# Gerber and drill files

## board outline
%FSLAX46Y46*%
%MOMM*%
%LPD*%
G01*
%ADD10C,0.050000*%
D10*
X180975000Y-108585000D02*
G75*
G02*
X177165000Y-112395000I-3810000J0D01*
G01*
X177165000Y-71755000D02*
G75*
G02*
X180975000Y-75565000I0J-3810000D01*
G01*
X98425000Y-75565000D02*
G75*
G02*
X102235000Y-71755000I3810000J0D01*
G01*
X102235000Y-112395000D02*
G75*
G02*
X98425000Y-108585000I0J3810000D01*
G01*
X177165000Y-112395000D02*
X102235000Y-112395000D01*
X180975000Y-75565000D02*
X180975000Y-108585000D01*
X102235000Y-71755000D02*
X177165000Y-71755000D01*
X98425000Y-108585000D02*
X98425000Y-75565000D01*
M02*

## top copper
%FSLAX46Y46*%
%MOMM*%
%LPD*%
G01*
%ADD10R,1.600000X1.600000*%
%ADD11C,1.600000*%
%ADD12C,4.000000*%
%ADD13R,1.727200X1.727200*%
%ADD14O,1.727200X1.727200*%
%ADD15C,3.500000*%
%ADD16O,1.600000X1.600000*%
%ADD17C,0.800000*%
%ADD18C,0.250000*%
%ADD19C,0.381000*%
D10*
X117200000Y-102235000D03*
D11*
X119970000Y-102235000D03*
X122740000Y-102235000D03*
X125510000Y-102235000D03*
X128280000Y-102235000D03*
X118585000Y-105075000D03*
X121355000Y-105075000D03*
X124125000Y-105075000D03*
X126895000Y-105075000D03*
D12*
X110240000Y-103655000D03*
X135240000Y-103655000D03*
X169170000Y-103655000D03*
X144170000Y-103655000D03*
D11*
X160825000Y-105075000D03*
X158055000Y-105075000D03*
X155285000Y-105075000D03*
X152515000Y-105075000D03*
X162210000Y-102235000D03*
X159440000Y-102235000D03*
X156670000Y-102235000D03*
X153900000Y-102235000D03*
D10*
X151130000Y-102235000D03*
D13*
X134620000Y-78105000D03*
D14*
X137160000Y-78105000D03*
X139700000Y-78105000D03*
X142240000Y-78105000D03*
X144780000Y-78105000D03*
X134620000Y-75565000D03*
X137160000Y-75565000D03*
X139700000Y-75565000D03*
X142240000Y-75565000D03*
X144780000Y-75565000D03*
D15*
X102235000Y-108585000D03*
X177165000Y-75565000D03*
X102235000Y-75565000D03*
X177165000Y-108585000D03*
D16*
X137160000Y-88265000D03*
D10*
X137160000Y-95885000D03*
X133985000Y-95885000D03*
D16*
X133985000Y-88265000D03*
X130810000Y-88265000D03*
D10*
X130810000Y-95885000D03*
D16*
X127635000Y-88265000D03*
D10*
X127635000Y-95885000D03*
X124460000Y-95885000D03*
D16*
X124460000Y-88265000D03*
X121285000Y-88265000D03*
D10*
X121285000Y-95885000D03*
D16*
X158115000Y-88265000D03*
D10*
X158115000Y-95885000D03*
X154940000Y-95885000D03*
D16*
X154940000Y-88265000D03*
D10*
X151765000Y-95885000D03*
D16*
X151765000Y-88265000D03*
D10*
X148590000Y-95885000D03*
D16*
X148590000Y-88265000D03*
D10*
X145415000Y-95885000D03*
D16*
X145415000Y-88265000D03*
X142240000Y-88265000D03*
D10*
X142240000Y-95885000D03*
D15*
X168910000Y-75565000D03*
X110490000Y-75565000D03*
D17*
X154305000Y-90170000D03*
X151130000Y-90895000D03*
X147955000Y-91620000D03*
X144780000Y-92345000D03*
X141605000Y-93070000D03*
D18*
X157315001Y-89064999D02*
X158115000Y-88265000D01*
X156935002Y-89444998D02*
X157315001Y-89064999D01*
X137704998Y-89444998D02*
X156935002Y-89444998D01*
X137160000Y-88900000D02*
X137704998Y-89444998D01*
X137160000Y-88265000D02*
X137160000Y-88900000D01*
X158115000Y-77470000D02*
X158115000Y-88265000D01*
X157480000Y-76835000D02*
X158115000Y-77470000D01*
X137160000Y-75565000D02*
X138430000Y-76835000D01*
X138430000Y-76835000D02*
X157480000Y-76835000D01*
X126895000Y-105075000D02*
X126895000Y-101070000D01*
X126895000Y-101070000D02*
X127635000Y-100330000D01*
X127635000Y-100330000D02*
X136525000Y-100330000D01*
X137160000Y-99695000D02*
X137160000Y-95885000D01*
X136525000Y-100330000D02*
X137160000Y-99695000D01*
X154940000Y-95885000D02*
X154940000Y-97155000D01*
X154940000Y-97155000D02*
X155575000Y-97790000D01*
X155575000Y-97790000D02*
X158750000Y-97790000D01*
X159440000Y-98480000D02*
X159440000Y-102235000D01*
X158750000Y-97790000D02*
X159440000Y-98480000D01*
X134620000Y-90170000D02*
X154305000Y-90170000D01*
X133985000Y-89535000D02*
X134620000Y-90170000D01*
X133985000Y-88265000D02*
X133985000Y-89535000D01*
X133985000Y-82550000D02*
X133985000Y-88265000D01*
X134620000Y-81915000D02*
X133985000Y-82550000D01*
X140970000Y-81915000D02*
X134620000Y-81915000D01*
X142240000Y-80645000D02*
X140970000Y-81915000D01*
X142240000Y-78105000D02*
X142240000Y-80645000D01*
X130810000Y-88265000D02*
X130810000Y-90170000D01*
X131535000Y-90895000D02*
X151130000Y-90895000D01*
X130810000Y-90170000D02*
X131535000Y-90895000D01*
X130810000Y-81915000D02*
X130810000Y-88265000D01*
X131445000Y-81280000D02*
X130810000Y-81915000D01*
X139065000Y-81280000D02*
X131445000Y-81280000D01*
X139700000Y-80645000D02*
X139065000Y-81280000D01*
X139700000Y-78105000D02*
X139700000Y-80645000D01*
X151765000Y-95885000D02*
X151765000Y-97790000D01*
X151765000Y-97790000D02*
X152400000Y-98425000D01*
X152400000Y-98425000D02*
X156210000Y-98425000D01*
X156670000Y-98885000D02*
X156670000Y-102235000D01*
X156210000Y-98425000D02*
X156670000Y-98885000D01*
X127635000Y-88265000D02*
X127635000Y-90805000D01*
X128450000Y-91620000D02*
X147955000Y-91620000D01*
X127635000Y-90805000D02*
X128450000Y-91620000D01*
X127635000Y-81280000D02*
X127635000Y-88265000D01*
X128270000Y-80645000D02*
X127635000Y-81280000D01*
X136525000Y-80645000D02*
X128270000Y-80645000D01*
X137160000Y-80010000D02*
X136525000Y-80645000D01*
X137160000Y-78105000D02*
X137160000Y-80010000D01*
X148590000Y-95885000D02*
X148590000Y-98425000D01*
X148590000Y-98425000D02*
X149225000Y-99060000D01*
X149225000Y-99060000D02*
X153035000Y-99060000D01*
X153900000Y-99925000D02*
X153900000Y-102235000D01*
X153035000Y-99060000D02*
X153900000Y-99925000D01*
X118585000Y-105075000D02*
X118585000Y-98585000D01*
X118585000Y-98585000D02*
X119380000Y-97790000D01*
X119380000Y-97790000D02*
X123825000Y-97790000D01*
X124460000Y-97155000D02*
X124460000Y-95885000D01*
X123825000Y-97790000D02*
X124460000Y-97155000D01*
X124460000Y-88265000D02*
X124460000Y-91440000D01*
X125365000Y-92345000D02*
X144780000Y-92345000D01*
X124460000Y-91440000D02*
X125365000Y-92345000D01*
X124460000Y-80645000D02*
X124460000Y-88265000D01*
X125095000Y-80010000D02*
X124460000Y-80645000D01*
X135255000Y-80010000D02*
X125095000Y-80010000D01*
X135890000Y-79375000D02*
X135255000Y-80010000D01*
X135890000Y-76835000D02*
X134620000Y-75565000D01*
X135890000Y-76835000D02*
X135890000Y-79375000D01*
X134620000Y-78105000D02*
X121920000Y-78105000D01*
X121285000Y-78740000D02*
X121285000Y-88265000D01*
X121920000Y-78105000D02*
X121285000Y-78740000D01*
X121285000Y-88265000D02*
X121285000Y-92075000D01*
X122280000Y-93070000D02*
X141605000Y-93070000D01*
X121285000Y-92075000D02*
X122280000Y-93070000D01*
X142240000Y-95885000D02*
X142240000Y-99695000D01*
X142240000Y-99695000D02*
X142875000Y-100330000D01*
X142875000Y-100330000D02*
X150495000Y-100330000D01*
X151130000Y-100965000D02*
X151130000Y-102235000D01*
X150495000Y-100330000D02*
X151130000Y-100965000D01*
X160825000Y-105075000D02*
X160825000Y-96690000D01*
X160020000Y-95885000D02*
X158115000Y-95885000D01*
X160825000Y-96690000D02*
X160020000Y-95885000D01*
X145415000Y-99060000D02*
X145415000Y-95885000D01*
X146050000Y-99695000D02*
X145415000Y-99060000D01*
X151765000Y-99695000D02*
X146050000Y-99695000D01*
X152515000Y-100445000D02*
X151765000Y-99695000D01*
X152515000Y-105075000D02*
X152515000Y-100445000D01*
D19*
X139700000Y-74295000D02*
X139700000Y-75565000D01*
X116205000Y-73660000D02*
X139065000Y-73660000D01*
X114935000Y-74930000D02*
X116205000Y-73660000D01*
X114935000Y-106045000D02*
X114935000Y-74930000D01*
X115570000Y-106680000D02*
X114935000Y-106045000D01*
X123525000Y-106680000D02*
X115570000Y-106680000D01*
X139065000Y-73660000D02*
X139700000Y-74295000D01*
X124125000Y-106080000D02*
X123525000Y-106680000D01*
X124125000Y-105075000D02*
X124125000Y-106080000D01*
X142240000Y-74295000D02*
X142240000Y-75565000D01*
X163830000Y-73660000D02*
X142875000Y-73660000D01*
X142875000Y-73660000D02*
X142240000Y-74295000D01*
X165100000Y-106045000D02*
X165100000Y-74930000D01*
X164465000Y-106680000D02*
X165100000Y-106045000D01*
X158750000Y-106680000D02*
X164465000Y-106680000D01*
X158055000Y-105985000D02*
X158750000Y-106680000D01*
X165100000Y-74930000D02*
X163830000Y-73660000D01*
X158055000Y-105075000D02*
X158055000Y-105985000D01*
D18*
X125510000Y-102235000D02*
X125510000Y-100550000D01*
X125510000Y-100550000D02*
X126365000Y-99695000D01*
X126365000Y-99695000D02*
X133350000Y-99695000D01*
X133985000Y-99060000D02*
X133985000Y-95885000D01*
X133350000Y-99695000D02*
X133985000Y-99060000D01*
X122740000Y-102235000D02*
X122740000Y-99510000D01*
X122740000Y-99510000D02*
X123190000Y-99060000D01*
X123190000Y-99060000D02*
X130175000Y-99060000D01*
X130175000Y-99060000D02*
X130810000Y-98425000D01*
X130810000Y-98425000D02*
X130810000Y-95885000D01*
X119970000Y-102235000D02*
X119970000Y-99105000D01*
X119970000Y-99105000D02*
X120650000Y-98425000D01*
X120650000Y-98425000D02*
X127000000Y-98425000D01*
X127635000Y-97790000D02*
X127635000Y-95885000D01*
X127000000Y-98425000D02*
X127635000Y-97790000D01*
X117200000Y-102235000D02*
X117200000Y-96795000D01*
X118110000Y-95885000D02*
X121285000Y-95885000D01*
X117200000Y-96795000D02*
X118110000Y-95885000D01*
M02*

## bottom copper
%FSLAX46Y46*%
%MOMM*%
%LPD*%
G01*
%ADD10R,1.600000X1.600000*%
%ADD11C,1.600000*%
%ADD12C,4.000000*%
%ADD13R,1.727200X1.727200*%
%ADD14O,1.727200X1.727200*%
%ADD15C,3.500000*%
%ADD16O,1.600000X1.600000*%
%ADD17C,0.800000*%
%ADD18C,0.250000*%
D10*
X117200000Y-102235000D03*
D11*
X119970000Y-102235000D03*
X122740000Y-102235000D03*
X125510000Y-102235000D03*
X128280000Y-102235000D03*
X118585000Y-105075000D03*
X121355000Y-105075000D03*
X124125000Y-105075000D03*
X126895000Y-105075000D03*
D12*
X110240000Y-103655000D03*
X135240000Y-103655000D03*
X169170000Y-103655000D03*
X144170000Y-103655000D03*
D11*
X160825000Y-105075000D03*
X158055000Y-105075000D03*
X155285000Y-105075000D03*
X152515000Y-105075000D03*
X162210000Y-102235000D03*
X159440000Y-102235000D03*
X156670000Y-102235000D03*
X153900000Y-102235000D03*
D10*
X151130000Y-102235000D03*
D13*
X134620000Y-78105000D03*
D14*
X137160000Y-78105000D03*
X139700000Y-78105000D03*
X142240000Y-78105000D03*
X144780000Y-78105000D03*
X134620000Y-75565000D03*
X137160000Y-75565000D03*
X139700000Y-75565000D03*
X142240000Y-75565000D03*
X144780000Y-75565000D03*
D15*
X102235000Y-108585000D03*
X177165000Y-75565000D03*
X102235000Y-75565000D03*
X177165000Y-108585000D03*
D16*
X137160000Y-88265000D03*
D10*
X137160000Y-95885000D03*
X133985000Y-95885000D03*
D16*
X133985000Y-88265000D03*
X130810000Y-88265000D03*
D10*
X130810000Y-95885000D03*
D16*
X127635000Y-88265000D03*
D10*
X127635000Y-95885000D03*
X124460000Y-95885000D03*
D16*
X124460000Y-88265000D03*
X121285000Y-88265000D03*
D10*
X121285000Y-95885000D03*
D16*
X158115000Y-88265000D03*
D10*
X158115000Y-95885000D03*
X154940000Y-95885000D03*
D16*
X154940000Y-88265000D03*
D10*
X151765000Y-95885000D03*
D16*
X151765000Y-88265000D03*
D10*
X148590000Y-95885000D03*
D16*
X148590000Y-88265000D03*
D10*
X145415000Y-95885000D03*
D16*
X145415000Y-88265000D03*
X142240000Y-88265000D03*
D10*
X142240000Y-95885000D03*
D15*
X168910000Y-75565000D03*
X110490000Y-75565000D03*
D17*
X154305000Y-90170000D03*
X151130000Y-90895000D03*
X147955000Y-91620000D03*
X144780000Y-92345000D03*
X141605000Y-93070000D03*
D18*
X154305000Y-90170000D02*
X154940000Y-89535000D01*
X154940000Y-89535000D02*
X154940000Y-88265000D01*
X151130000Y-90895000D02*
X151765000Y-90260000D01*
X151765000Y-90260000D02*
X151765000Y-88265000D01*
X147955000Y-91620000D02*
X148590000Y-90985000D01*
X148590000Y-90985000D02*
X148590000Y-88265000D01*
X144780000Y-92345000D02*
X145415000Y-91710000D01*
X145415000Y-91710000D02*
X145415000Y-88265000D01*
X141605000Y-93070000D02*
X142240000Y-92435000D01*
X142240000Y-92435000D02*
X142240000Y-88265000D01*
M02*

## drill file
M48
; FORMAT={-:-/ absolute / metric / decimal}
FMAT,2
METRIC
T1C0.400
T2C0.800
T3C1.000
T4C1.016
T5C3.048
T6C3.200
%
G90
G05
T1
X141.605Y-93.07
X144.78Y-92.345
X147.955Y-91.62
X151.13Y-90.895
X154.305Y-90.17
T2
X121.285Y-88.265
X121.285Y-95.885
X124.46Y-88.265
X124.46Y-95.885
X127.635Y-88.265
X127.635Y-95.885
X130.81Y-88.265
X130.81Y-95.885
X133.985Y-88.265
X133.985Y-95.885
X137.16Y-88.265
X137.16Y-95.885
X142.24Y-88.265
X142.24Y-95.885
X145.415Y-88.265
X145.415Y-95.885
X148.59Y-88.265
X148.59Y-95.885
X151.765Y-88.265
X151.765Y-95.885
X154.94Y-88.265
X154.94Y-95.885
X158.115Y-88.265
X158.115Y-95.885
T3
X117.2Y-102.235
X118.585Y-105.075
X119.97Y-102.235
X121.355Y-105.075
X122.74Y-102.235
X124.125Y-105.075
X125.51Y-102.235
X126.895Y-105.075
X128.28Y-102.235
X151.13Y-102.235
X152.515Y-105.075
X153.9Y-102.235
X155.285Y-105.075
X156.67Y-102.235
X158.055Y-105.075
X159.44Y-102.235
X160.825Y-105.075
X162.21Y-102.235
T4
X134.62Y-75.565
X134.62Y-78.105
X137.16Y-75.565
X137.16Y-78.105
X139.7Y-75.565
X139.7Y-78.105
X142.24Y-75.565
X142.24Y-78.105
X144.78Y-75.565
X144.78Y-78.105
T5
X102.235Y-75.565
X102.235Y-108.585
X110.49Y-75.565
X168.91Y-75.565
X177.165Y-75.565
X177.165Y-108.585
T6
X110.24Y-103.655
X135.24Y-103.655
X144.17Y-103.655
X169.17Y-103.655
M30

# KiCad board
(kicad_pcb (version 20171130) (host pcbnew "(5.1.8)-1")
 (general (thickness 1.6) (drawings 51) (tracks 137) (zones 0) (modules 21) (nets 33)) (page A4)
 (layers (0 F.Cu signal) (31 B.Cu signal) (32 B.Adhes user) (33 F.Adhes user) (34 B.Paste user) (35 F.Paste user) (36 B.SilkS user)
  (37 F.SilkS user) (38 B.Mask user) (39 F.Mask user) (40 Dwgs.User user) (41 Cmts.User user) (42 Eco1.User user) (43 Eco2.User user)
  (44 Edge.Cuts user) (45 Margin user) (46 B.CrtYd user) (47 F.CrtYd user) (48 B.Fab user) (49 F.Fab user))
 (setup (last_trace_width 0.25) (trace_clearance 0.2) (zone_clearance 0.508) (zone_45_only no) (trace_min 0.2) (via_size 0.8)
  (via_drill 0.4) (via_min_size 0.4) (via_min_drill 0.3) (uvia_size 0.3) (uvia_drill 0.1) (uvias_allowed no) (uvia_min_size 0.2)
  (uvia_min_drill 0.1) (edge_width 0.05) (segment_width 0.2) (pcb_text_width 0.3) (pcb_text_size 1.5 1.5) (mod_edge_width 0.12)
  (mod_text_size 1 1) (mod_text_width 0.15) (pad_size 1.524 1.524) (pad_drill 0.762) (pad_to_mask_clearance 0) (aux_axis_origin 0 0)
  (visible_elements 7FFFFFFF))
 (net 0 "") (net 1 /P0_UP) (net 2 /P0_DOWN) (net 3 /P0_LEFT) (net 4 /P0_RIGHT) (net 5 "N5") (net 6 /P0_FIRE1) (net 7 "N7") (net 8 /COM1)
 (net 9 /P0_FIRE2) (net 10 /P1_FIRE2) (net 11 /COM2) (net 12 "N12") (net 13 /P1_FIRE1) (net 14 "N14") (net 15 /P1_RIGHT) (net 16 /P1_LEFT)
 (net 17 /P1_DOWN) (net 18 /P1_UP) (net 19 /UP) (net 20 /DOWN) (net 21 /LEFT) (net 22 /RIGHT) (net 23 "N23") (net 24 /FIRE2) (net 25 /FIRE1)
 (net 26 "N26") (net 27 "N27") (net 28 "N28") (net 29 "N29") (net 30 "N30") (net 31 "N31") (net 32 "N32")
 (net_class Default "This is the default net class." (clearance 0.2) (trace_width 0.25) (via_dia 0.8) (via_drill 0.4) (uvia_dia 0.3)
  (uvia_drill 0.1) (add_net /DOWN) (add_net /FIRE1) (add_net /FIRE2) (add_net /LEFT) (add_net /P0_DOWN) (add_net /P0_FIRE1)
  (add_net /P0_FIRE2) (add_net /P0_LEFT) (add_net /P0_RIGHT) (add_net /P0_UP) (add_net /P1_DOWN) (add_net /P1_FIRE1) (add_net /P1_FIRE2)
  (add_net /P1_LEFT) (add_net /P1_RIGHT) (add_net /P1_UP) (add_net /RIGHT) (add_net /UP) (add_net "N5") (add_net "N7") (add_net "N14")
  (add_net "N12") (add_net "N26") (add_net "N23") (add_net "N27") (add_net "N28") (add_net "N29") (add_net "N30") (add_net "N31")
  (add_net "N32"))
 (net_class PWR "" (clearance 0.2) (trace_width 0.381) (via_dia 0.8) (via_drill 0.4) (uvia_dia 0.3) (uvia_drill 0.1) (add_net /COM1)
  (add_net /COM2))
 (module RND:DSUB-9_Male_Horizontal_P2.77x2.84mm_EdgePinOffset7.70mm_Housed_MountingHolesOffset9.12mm (layer F.Cu) (at 117.2 102.235)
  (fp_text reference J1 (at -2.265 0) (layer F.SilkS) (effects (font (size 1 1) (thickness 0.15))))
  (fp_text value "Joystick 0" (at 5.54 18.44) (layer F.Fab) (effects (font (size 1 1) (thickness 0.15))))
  (pad 1 thru_hole rect (at 0 0) (size 1.6 1.6) (drill 1) (layers *.Cu *.Mask) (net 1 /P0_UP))
  (pad 2 thru_hole circle (at 2.77 0) (size 1.6 1.6) (drill 1) (layers *.Cu *.Mask) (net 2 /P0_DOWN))
  (pad 3 thru_hole circle (at 5.54 0) (size 1.6 1.6) (drill 1) (layers *.Cu *.Mask) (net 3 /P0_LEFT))
  (pad 4 thru_hole circle (at 8.31 0) (size 1.6 1.6) (drill 1) (layers *.Cu *.Mask) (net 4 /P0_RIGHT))
  (pad 5 thru_hole circle (at 11.08 0) (size 1.6 1.6) (drill 1) (layers *.Cu *.Mask) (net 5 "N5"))
  (pad 6 thru_hole circle (at 1.385 2.84) (size 1.6 1.6) (drill 1) (layers *.Cu *.Mask) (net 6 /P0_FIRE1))
  (pad 7 thru_hole circle (at 4.155 2.84) (size 1.6 1.6) (drill 1) (layers *.Cu *.Mask) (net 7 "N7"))
  (pad 8 thru_hole circle (at 6.925 2.84) (size 1.6 1.6) (drill 1) (layers *.Cu *.Mask) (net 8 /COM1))
  (pad 9 thru_hole circle (at 9.695 2.84) (size 1.6 1.6) (drill 1) (layers *.Cu *.Mask) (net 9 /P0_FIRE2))
  (pad 0 thru_hole circle (at -6.96 1.42) (size 4 4) (drill 3.2) (layers *.Cu *.Mask))
  (pad 0 thru_hole circle (at 18.04 1.42) (size 4 4) (drill 3.2) (layers *.Cu *.Mask)))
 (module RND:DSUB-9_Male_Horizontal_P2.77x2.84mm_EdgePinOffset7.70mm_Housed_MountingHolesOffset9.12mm (layer F.Cu) (at 151.13 102.235)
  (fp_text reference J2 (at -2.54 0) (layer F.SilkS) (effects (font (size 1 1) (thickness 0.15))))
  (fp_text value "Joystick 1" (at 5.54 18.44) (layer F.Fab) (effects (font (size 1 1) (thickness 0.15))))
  (pad 0 thru_hole circle (at 18.04 1.42) (size 4 4) (drill 3.2) (layers *.Cu *.Mask))
  (pad 0 thru_hole circle (at -6.96 1.42) (size 4 4) (drill 3.2) (layers *.Cu *.Mask))
  (pad 9 thru_hole circle (at 9.695 2.84) (size 1.6 1.6) (drill 1) (layers *.Cu *.Mask) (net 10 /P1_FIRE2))
  (pad 8 thru_hole circle (at 6.925 2.84) (size 1.6 1.6) (drill 1) (layers *.Cu *.Mask) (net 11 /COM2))
  (pad 7 thru_hole circle (at 4.155 2.84) (size 1.6 1.6) (drill 1) (layers *.Cu *.Mask) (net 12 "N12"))
  (pad 6 thru_hole circle (at 1.385 2.84) (size 1.6 1.6) (drill 1) (layers *.Cu *.Mask) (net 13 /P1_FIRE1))
  (pad 5 thru_hole circle (at 11.08 0) (size 1.6 1.6) (drill 1) (layers *.Cu *.Mask) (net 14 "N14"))
  (pad 4 thru_hole circle (at 8.31 0) (size 1.6 1.6) (drill 1) (layers *.Cu *.Mask) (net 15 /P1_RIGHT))
  (pad 3 thru_hole circle (at 5.54 0) (size 1.6 1.6) (drill 1) (layers *.Cu *.Mask) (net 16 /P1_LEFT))
  (pad 2 thru_hole circle (at 2.77 0) (size 1.6 1.6) (drill 1) (layers *.Cu *.Mask) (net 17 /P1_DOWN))
  (pad 1 thru_hole rect (at 0 0) (size 1.6 1.6) (drill 1) (layers *.Cu *.Mask) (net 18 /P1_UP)))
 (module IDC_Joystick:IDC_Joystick (layer F.Cu) (at 134.62 78.105 90)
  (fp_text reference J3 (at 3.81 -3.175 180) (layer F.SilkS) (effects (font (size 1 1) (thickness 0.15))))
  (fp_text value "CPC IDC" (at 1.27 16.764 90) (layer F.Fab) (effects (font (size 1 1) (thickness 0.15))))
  (pad 1 thru_hole rect (at 0 0 90) (size 1.7272 1.7272) (drill 1.016) (layers *.Cu *.Mask) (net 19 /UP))
  (pad 2 thru_hole oval (at 0 2.54 90) (size 1.7272 1.7272) (drill 1.016) (layers *.Cu *.Mask) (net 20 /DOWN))
  (pad 3 thru_hole oval (at 0 5.08 90) (size 1.7272 1.7272) (drill 1.016) (layers *.Cu *.Mask) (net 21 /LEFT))
  (pad 4 thru_hole oval (at 0 7.62 90) (size 1.7272 1.7272) (drill 1.016) (layers *.Cu *.Mask) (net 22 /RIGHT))
  (pad 5 thru_hole oval (at 0 10.16 90) (size 1.7272 1.7272) (drill 1.016) (layers *.Cu *.Mask) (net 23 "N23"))
  (pad 6 thru_hole oval (at 2.54 0 90) (size 1.7272 1.7272) (drill 1.016) (layers *.Cu *.Mask) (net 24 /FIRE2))
  (pad 7 thru_hole oval (at 2.54 2.54 90) (size 1.7272 1.7272) (drill 1.016) (layers *.Cu *.Mask) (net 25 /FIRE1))
  (pad 8 thru_hole oval (at 2.54 5.08 90) (size 1.7272 1.7272) (drill 1.016) (layers *.Cu *.Mask) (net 8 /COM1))
  (pad 9 thru_hole oval (at 2.54 7.62 90) (size 1.7272 1.7272) (drill 1.016) (layers *.Cu *.Mask) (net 11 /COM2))
  (pad 10 thru_hole oval (at 2.54 10.16 90) (size 1.7272 1.7272) (drill 1.016) (layers *.Cu *.Mask) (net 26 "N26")))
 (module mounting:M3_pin (layer F.Cu) (at 102.235 108.585)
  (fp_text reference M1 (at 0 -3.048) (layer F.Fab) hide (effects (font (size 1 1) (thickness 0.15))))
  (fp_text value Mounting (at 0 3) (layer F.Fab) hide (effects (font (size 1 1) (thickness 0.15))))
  (pad 1 thru_hole circle (at 0 0) (size 3.5 3.5) (drill 3.048) (layers *.Cu *.Mask) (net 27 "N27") (solder_mask_margin 0.8)))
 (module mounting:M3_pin (layer F.Cu) (at 177.165 75.565)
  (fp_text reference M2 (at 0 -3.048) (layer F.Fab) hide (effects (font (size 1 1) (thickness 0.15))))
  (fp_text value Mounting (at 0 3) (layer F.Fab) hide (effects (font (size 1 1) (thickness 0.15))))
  (pad 1 thru_hole circle (at 0 0) (size 3.5 3.5) (drill 3.048) (layers *.Cu *.Mask) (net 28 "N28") (solder_mask_margin 0.8)))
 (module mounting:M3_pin (layer F.Cu) (at 102.235 75.565)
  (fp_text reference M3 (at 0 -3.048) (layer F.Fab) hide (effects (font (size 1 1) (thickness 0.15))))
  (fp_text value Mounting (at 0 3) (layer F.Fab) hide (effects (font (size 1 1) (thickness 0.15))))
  (pad 1 thru_hole circle (at 0 0) (size 3.5 3.5) (drill 3.048) (layers *.Cu *.Mask) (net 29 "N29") (solder_mask_margin 0.8)))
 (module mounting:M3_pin (layer F.Cu) (at 177.165 108.585)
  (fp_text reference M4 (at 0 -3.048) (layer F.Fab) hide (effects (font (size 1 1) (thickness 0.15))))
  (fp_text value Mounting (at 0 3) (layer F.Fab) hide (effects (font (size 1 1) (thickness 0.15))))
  (pad 1 thru_hole circle (at 0 0) (size 3.5 3.5) (drill 3.048) (layers *.Cu *.Mask) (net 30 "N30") (solder_mask_margin 0.8)))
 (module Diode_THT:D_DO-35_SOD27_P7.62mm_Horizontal (layer F.Cu) (at 137.16 95.885 90)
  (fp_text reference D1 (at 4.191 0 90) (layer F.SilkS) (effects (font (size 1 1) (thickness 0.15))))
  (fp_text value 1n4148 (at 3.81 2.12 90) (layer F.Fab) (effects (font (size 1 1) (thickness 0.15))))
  (pad 2 thru_hole oval (at 7.62 0 90) (size 1.6 1.6) (drill 0.8) (layers *.Cu *.Mask) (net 25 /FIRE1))
  (pad 1 thru_hole rect (at 0 0 90) (size 1.6 1.6) (drill 0.8) (layers *.Cu *.Mask) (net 9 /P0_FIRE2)))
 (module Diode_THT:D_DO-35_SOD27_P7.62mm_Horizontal (layer F.Cu) (at 133.985 95.885 90)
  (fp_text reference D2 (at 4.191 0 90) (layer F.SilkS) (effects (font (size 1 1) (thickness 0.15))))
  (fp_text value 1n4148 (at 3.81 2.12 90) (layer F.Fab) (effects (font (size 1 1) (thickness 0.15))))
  (pad 1 thru_hole rect (at 0 0 90) (size 1.6 1.6) (drill 0.8) (layers *.Cu *.Mask) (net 4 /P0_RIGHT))
  (pad 2 thru_hole oval (at 7.62 0 90) (size 1.6 1.6) (drill 0.8) (layers *.Cu *.Mask) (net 22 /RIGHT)))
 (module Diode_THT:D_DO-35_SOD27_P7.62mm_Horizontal (layer F.Cu) (at 130.81 95.885 90)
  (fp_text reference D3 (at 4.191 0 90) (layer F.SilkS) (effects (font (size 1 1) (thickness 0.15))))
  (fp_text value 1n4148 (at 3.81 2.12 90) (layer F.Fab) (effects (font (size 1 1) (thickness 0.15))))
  (pad 2 thru_hole oval (at 7.62 0 90) (size 1.6 1.6) (drill 0.8) (layers *.Cu *.Mask) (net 21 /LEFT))
  (pad 1 thru_hole rect (at 0 0 90) (size 1.6 1.6) (drill 0.8) (layers *.Cu *.Mask) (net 3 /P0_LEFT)))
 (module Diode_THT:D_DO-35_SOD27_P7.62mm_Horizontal (layer F.Cu) (at 127.635 95.885 90)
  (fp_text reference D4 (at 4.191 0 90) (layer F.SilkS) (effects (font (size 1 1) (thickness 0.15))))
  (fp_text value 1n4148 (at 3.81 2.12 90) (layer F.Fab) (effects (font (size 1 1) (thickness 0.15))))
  (pad 2 thru_hole oval (at 7.62 0 90) (size 1.6 1.6) (drill 0.8) (layers *.Cu *.Mask) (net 20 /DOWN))
  (pad 1 thru_hole rect (at 0 0 90) (size 1.6 1.6) (drill 0.8) (layers *.Cu *.Mask) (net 2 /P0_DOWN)))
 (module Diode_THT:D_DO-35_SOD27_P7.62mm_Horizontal (layer F.Cu) (at 124.46 95.885 90)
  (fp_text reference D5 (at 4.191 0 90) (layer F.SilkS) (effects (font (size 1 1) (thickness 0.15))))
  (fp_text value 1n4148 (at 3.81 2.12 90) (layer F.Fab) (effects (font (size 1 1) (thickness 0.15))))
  (pad 1 thru_hole rect (at 0 0 90) (size 1.6 1.6) (drill 0.8) (layers *.Cu *.Mask) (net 6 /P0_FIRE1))
  (pad 2 thru_hole oval (at 7.62 0 90) (size 1.6 1.6) (drill 0.8) (layers *.Cu *.Mask) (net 24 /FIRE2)))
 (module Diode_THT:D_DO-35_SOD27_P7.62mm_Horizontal (layer F.Cu) (at 121.285 95.885 90)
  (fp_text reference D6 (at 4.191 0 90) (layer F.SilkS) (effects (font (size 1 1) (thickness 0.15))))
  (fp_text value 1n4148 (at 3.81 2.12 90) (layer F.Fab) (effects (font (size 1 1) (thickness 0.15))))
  (pad 2 thru_hole oval (at 7.62 0 90) (size 1.6 1.6) (drill 0.8) (layers *.Cu *.Mask) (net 19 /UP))
  (pad 1 thru_hole rect (at 0 0 90) (size 1.6 1.6) (drill 0.8) (layers *.Cu *.Mask) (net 1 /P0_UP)))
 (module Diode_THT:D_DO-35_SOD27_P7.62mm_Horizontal (layer F.Cu) (at 158.115 95.885 90)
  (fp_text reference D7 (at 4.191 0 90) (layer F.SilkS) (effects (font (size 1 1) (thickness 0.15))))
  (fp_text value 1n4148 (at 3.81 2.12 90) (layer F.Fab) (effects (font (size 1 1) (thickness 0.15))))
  (pad 2 thru_hole oval (at 7.62 0 90) (size 1.6 1.6) (drill 0.8) (layers *.Cu *.Mask) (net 25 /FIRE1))
  (pad 1 thru_hole rect (at 0 0 90) (size 1.6 1.6) (drill 0.8) (layers *.Cu *.Mask) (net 10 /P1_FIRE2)))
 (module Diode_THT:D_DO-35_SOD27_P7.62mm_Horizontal (layer F.Cu) (at 154.94 95.885 90)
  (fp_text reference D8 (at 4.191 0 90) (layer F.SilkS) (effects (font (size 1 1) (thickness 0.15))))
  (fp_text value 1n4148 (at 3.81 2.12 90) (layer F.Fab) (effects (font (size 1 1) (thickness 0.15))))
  (pad 1 thru_hole rect (at 0 0 90) (size 1.6 1.6) (drill 0.8) (layers *.Cu *.Mask) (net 15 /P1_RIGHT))
  (pad 2 thru_hole oval (at 7.62 0 90) (size 1.6 1.6) (drill 0.8) (layers *.Cu *.Mask) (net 22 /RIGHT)))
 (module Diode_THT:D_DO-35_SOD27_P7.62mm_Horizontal (layer F.Cu) (at 151.765 95.885 90)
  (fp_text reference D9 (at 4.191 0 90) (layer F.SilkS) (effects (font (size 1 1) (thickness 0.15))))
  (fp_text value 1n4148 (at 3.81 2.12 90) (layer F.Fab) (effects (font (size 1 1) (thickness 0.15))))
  (pad 1 thru_hole rect (at 0 0 90) (size 1.6 1.6) (drill 0.8) (layers *.Cu *.Mask) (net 16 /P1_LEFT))
  (pad 2 thru_hole oval (at 7.62 0 90) (size 1.6 1.6) (drill 0.8) (layers *.Cu *.Mask) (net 21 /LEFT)))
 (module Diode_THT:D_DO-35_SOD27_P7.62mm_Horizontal (layer F.Cu) (at 148.59 95.885 90)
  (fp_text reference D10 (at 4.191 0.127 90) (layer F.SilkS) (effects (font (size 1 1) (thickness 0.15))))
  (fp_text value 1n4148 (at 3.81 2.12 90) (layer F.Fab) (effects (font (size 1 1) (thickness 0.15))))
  (pad 1 thru_hole rect (at 0 0 90) (size 1.6 1.6) (drill 0.8) (layers *.Cu *.Mask) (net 17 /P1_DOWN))
  (pad 2 thru_hole oval (at 7.62 0 90) (size 1.6 1.6) (drill 0.8) (layers *.Cu *.Mask) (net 20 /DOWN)))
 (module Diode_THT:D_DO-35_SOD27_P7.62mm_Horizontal (layer F.Cu) (at 145.415 95.885 90)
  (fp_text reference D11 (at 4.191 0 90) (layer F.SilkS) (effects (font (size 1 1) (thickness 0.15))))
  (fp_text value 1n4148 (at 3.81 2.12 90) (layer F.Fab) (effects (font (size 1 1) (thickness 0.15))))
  (pad 1 thru_hole rect (at 0 0 90) (size 1.6 1.6) (drill 0.8) (layers *.Cu *.Mask) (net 13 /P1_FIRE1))
  (pad 2 thru_hole oval (at 7.62 0 90) (size 1.6 1.6) (drill 0.8) (layers *.Cu *.Mask) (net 24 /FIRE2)))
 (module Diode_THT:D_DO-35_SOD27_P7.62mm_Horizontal (layer F.Cu) (at 142.24 95.885 90)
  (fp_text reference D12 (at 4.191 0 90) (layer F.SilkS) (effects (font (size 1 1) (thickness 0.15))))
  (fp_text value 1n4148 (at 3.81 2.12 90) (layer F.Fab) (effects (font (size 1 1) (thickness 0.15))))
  (pad 2 thru_hole oval (at 7.62 0 90) (size 1.6 1.6) (drill 0.8) (layers *.Cu *.Mask) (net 19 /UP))
  (pad 1 thru_hole rect (at 0 0 90) (size 1.6 1.6) (drill 0.8) (layers *.Cu *.Mask) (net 18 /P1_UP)))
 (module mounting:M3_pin (layer F.Cu) (at 168.91 75.565)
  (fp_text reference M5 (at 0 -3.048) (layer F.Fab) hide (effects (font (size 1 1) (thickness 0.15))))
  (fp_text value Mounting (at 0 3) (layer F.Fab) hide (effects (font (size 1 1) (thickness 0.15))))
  (pad 1 thru_hole circle (at 0 0) (size 3.5 3.5) (drill 3.048) (layers *.Cu *.Mask) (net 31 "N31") (solder_mask_margin 0.8)))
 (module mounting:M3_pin (layer F.Cu) (at 110.49 75.565)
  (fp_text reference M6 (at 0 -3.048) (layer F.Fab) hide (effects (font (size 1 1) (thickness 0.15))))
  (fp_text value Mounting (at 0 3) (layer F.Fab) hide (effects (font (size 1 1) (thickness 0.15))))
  (pad 1 thru_hole circle (at 0 0) (size 3.5 3.5) (drill 3.048) (layers *.Cu *.Mask) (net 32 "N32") (solder_mask_margin 0.8)))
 (gr_arc (start 177.165 108.585) (end 177.165 112.395) (angle -90) (layer Edge.Cuts) (width 0.05))
 (gr_arc (start 177.165 75.565) (end 180.975 75.565) (angle -90) (layer Edge.Cuts) (width 0.05))
 (gr_arc (start 102.235 75.565) (end 102.235 71.755) (angle -90) (layer Edge.Cuts) (width 0.05))
 (gr_arc (start 102.235 108.585) (end 98.425 108.585) (angle -90) (layer Edge.Cuts) (width 0.05))
 (gr_line (start 177.165 112.395) (end 102.235 112.395) (layer Edge.Cuts) (width 0.05))
 (gr_line (start 180.975 75.565) (end 180.975 108.585) (layer Edge.Cuts) (width 0.05))
 (gr_line (start 102.235 71.755) (end 177.165 71.755) (layer Edge.Cuts) (width 0.05))
 (gr_line (start 98.425 108.585) (end 98.425 75.565) (layer Edge.Cuts) (width 0.05))
 (segment (start 157.315001 89.064999) (end 158.115 88.265) (width 0.25) (layer F.Cu) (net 25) (status 20))
 (segment (start 156.935002 89.444998) (end 157.315001 89.064999) (width 0.25) (layer F.Cu) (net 25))
 (segment (start 137.704998 89.444998) (end 156.935002 89.444998) (width 0.25) (layer F.Cu) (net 25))
 (segment (start 137.16 88.9) (end 137.704998 89.444998) (width 0.25) (layer F.Cu) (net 25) (status 10))
 (segment (start 137.16 88.265) (end 137.16 88.9) (width 0.25) (layer F.Cu) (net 25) (status 30))
 (segment (start 158.115 77.47) (end 158.115 88.265) (width 0.25) (layer F.Cu) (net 25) (status 20))
 (segment (start 157.48 76.835) (end 158.115 77.47) (width 0.25) (layer F.Cu) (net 25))
 (segment (start 137.16 75.565) (end 138.43 76.835) (width 0.25) (layer F.Cu) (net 25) (status 10))
 (segment (start 138.43 76.835) (end 157.48 76.835) (width 0.25) (layer F.Cu) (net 25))
 (segment (start 126.895 105.075) (end 126.895 101.07) (width 0.25) (layer F.Cu) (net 9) (status 10))
 (segment (start 126.895 101.07) (end 127.635 100.33) (width 0.25) (layer F.Cu) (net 9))
 (segment (start 127.635 100.33) (end 136.525 100.33) (width 0.25) (layer F.Cu) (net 9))
 (segment (start 137.16 99.695) (end 137.16 95.885) (width 0.25) (layer F.Cu) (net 9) (status 20))
 (segment (start 136.525 100.33) (end 137.16 99.695) (width 0.25) (layer F.Cu) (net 9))
 (segment (start 154.94 95.885) (end 154.94 97.155) (width 0.25) (layer F.Cu) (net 15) (status 10))
 (segment (start 154.94 97.155) (end 155.575 97.79) (width 0.25) (layer F.Cu) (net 15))
 (segment (start 155.575 97.79) (end 158.75 97.79) (width 0.25) (layer F.Cu) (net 15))
 (segment (start 159.44 98.48) (end 159.44 102.235) (width 0.25) (layer F.Cu) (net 15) (status 20))
 (segment (start 158.75 97.79) (end 159.44 98.48) (width 0.25) (layer F.Cu) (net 15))
 (via (at 154.305 90.17) (size 0.8) (drill 0.4) (layers F.Cu B.Cu) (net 22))
 (segment (start 154.305 90.17) (end 154.94 89.535) (width 0.25) (layer B.Cu) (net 22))
 (segment (start 154.94 89.535) (end 154.94 88.265) (width 0.25) (layer B.Cu) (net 22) (status 20))
 (segment (start 134.62 90.17) (end 154.305 90.17) (width 0.25) (layer F.Cu) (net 22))
 (segment (start 133.985 89.535) (end 134.62 90.17) (width 0.25) (layer F.Cu) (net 22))
 (segment (start 133.985 88.265) (end 133.985 89.535) (width 0.25) (layer F.Cu) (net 22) (status 10))
 (segment (start 133.985 82.55) (end 133.985 88.265) (width 0.25) (layer F.Cu) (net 22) (status 20))
 (segment (start 134.62 81.915) (end 133.985 82.55) (width 0.25) (layer F.Cu) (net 22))
 (segment (start 140.97 81.915) (end 134.62 81.915) (width 0.25) (layer F.Cu) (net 22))
 (segment (start 142.24 80.645) (end 140.97 81.915) (width 0.25) (layer F.Cu) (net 22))
 (segment (start 142.24 78.105) (end 142.24 80.645) (width 0.25) (layer F.Cu) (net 22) (status 10))
 (segment (start 130.81 88.265) (end 130.81 90.17) (width 0.25) (layer F.Cu) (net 21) (status 10))
 (via (at 151.13 90.895) (size 0.8) (drill 0.4) (layers F.Cu B.Cu) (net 21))
 (segment (start 131.535 90.895) (end 151.13 90.895) (width 0.25) (layer F.Cu) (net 21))
 (segment (start 130.81 90.17) (end 131.535 90.895) (width 0.25) (layer F.Cu) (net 21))
 (segment (start 151.13 90.895) (end 151.765 90.26) (width 0.25) (layer B.Cu) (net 21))
 (segment (start 151.765 90.26) (end 151.765 88.265) (width 0.25) (layer B.Cu) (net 21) (status 20))
 (segment (start 130.81 81.915) (end 130.81 88.265) (width 0.25) (layer F.Cu) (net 21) (status 20))
 (segment (start 131.445 81.28) (end 130.81 81.915) (width 0.25) (layer F.Cu) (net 21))
 (segment (start 139.065 81.28) (end 131.445 81.28) (width 0.25) (layer F.Cu) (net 21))
 (segment (start 139.7 80.645) (end 139.065 81.28) (width 0.25) (layer F.Cu) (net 21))
 (segment (start 139.7 78.105) (end 139.7 80.645) (width 0.25) (layer F.Cu) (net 21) (status 10))
 (segment (start 151.765 95.885) (end 151.765 97.79) (width 0.25) (layer F.Cu) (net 16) (status 10))
 (segment (start 151.765 97.79) (end 152.4 98.425) (width 0.25) (layer F.Cu) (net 16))
 (segment (start 152.4 98.425) (end 156.21 98.425) (width 0.25) (layer F.Cu) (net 16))
 (segment (start 156.67 98.885) (end 156.67 102.235) (width 0.25) (layer F.Cu) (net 16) (status 20))
 (segment (start 156.21 98.425) (end 156.67 98.885) (width 0.25) (layer F.Cu) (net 16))
 (segment (start 127.635 88.265) (end 127.635 90.805) (width 0.25) (layer F.Cu) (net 20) (status 10))
 (via (at 147.955 91.62) (size 0.8) (drill 0.4) (layers F.Cu B.Cu) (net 20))
 (segment (start 128.45 91.62) (end 147.955 91.62) (width 0.25) (layer F.Cu) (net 20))
 (segment (start 127.635 90.805) (end 128.45 91.62) (width 0.25) (layer F.Cu) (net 20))
 (segment (start 147.955 91.62) (end 148.59 90.985) (width 0.25) (layer B.Cu) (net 20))
 (segment (start 148.59 90.985) (end 148.59 88.265) (width 0.25) (layer B.Cu) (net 20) (status 20))
 (segment (start 127.635 81.28) (end 127.635 88.265) (width 0.25) (layer F.Cu) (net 20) (status 20))
 (segment (start 128.27 80.645) (end 127.635 81.28) (width 0.25) (layer F.Cu) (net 20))
 (segment (start 136.525 80.645) (end 128.27 80.645) (width 0.25) (layer F.Cu) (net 20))
 (segment (start 137.16 80.01) (end 136.525 80.645) (width 0.25) (layer F.Cu) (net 20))
 (segment (start 137.16 78.105) (end 137.16 80.01) (width 0.25) (layer F.Cu) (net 20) (status 10))
 (segment (start 148.59 95.885) (end 148.59 98.425) (width 0.25) (layer F.Cu) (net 17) (status 10))
 (segment (start 148.59 98.425) (end 149.225 99.06) (width 0.25) (layer F.Cu) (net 17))
 (segment (start 149.225 99.06) (end 153.035 99.06) (width 0.25) (layer F.Cu) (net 17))
 (segment (start 153.9 99.925) (end 153.9 102.235) (width 0.25) (layer F.Cu) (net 17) (status 20))
 (segment (start 153.035 99.06) (end 153.9 99.925) (width 0.25) (layer F.Cu) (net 17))
 (segment (start 118.585 105.075) (end 118.585 98.585) (width 0.25) (layer F.Cu) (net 6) (status 10))
 (segment (start 118.585 98.585) (end 119.38 97.79) (width 0.25) (layer F.Cu) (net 6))
 (segment (start 119.38 97.79) (end 123.825 97.79) (width 0.25) (layer F.Cu) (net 6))
 (segment (start 124.46 97.155) (end 124.46 95.885) (width 0.25) (layer F.Cu) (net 6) (status 20))
 (segment (start 123.825 97.79) (end 124.46 97.155) (width 0.25) (layer F.Cu) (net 6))
 (segment (start 124.46 88.265) (end 124.46 91.44) (width 0.25) (layer F.Cu) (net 24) (status 10))
 (via (at 144.78 92.345) (size 0.8) (drill 0.4) (layers F.Cu B.Cu) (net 24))
 (segment (start 125.365 92.345) (end 144.78 92.345) (width 0.25) (layer F.Cu) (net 24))
 (segment (start 124.46 91.44) (end 125.365 92.345) (width 0.25) (layer F.Cu) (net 24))
 (segment (start 144.78 92.345) (end 145.415 91.71) (width 0.25) (layer B.Cu) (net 24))
 (segment (start 145.415 91.71) (end 145.415 88.265) (width 0.25) (layer B.Cu) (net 24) (status 20))
 (segment (start 124.46 80.645) (end 124.46 88.265) (width 0.25) (layer F.Cu) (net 24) (status 20))
 (segment (start 125.095 80.01) (end 124.46 80.645) (width 0.25) (layer F.Cu) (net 24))
 (segment (start 135.255 80.01) (end 125.095 80.01) (width 0.25) (layer F.Cu) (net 24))
 (segment (start 135.89 79.375) (end 135.255 80.01) (width 0.25) (layer F.Cu) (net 24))
 (segment (start 135.89 76.835) (end 134.62 75.565) (width 0.25) (layer F.Cu) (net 24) (status 20))
 (segment (start 135.89 76.835) (end 135.89 79.375) (width 0.25) (layer F.Cu) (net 24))
 (segment (start 134.62 78.105) (end 121.92 78.105) (width 0.25) (layer F.Cu) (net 19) (status 10))
 (segment (start 121.285 78.74) (end 121.285 88.265) (width 0.25) (layer F.Cu) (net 19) (status 20))
 (segment (start 121.92 78.105) (end 121.285 78.74) (width 0.25) (layer F.Cu) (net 19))
 (segment (start 121.285 88.265) (end 121.285 92.075) (width 0.25) (layer F.Cu) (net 19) (status 10))
 (via (at 141.605 93.07) (size 0.8) (drill 0.4) (layers F.Cu B.Cu) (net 19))
 (segment (start 122.28 93.07) (end 141.605 93.07) (width 0.25) (layer F.Cu) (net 19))
 (segment (start 121.285 92.075) (end 122.28 93.07) (width 0.25) (layer F.Cu) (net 19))
 (segment (start 141.605 93.07) (end 142.24 92.435) (width 0.25) (layer B.Cu) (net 19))
 (segment (start 142.24 92.435) (end 142.24 88.265) (width 0.25) (layer B.Cu) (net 19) (status 20))
 (segment (start 142.24 95.885) (end 142.24 99.695) (width 0.25) (layer F.Cu) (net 18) (status 10))
 (segment (start 142.24 99.695) (end 142.875 100.33) (width 0.25) (layer F.Cu) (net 18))
 (segment (start 142.875 100.33) (end 150.495 100.33) (width 0.25) (layer F.Cu) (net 18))
 (segment (start 151.13 100.965) (end 151.13 102.235) (width 0.25) (layer F.Cu) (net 18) (status 20))
 (segment (start 150.495 100.33) (end 151.13 100.965) (width 0.25) (layer F.Cu) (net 18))
 (segment (start 160.825 105.075) (end 160.825 96.69) (width 0.25) (layer F.Cu) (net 10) (status 10))
 (segment (start 160.02 95.885) (end 158.115 95.885) (width 0.25) (layer F.Cu) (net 10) (status 20))
 (segment (start 160.825 96.69) (end 160.02 95.885) (width 0.25) (layer F.Cu) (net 10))
 (segment (start 145.415 99.06) (end 145.415 95.885) (width 0.25) (layer F.Cu) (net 13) (status 20))
 (segment (start 146.05 99.695) (end 145.415 99.06) (width 0.25) (layer F.Cu) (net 13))
 (segment (start 151.765 99.695) (end 146.05 99.695) (width 0.25) (layer F.Cu) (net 13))
 (segment (start 152.515 100.445) (end 151.765 99.695) (width 0.25) (layer F.Cu) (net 13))
 (segment (start 152.515 105.075) (end 152.515 100.445) (width 0.25) (layer F.Cu) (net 13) (status 10))
 (segment (start 139.7 74.295) (end 139.7 75.565) (width 0.381) (layer F.Cu) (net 8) (status 20))
 (segment (start 116.205 73.66) (end 139.065 73.66) (width 0.381) (layer F.Cu) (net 8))
 (segment (start 114.935 74.93) (end 116.205 73.66) (width 0.381) (layer F.Cu) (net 8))
 (segment (start 114.935 106.045) (end 114.935 74.93) (width 0.381) (layer F.Cu) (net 8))
 (segment (start 115.57 106.68) (end 114.935 106.045) (width 0.381) (layer F.Cu) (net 8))
 (segment (start 123.525 106.68) (end 115.57 106.68) (width 0.381) (layer F.Cu) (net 8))
 (segment (start 139.065 73.66) (end 139.7 74.295) (width 0.381) (layer F.Cu) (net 8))
 (segment (start 124.125 106.08) (end 123.525 106.68) (width 0.381) (layer F.Cu) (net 8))
 (segment (start 124.125 105.075) (end 124.125 106.08) (width 0.381) (layer F.Cu) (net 8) (status 10))
 (segment (start 142.24 74.295) (end 142.24 75.565) (width 0.381) (layer F.Cu) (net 11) (status 20))
 (segment (start 163.83 73.66) (end 142.875 73.66) (width 0.381) (layer F.Cu) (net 11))
 (segment (start 142.875 73.66) (end 142.24 74.295) (width 0.381) (layer F.Cu) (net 11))
 (segment (start 165.1 106.045) (end 165.1 74.93) (width 0.381) (layer F.Cu) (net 11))
 (segment (start 164.465 106.68) (end 165.1 106.045) (width 0.381) (layer F.Cu) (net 11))
 (segment (start 158.75 106.68) (end 164.465 106.68) (width 0.381) (layer F.Cu) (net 11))
 (segment (start 158.055 105.985) (end 158.75 106.68) (width 0.381) (layer F.Cu) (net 11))
 (segment (start 165.1 74.93) (end 163.83 73.66) (width 0.381) (layer F.Cu) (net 11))
 (segment (start 158.055 105.075) (end 158.055 105.985) (width 0.381) (layer F.Cu) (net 11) (status 10))
 (segment (start 125.51 102.235) (end 125.51 100.55) (width 0.25) (layer F.Cu) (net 4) (status 10))
 (segment (start 125.51 100.55) (end 126.365 99.695) (width 0.25) (layer F.Cu) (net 4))
 (segment (start 126.365 99.695) (end 133.35 99.695) (width 0.25) (layer F.Cu) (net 4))
 (segment (start 133.985 99.06) (end 133.985 95.885) (width 0.25) (layer F.Cu) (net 4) (status 20))
 (segment (start 133.35 99.695) (end 133.985 99.06) (width 0.25) (layer F.Cu) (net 4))
 (segment (start 122.74 102.235) (end 122.74 99.51) (width 0.25) (layer F.Cu) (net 3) (status 10))
 (segment (start 122.74 99.51) (end 123.19 99.06) (width 0.25) (layer F.Cu) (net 3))
 (segment (start 123.19 99.06) (end 130.175 99.06) (width 0.25) (layer F.Cu) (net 3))
 (segment (start 130.175 99.06) (end 130.81 98.425) (width 0.25) (layer F.Cu) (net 3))
 (segment (start 130.81 98.425) (end 130.81 95.885) (width 0.25) (layer F.Cu) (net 3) (status 20))
 (segment (start 119.97 102.235) (end 119.97 99.105) (width 0.25) (layer F.Cu) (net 2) (status 10))
 (segment (start 119.97 99.105) (end 120.65 98.425) (width 0.25) (layer F.Cu) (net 2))
 (segment (start 120.65 98.425) (end 127 98.425) (width 0.25) (layer F.Cu) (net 2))
 (segment (start 127.635 97.79) (end 127.635 95.885) (width 0.25) (layer F.Cu) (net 2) (status 20))
 (segment (start 127 98.425) (end 127.635 97.79) (width 0.25) (layer F.Cu) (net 2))
 (segment (start 117.2 102.235) (end 117.2 96.795) (width 0.25) (layer F.Cu) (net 1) (status 10))
 (segment (start 118.11 95.885) (end 121.285 95.885) (width 0.25) (layer F.Cu) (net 1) (status 20))
 (segment (start 117.2 96.795) (end 118.11 95.885) (width 0.25) (layer F.Cu) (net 1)))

